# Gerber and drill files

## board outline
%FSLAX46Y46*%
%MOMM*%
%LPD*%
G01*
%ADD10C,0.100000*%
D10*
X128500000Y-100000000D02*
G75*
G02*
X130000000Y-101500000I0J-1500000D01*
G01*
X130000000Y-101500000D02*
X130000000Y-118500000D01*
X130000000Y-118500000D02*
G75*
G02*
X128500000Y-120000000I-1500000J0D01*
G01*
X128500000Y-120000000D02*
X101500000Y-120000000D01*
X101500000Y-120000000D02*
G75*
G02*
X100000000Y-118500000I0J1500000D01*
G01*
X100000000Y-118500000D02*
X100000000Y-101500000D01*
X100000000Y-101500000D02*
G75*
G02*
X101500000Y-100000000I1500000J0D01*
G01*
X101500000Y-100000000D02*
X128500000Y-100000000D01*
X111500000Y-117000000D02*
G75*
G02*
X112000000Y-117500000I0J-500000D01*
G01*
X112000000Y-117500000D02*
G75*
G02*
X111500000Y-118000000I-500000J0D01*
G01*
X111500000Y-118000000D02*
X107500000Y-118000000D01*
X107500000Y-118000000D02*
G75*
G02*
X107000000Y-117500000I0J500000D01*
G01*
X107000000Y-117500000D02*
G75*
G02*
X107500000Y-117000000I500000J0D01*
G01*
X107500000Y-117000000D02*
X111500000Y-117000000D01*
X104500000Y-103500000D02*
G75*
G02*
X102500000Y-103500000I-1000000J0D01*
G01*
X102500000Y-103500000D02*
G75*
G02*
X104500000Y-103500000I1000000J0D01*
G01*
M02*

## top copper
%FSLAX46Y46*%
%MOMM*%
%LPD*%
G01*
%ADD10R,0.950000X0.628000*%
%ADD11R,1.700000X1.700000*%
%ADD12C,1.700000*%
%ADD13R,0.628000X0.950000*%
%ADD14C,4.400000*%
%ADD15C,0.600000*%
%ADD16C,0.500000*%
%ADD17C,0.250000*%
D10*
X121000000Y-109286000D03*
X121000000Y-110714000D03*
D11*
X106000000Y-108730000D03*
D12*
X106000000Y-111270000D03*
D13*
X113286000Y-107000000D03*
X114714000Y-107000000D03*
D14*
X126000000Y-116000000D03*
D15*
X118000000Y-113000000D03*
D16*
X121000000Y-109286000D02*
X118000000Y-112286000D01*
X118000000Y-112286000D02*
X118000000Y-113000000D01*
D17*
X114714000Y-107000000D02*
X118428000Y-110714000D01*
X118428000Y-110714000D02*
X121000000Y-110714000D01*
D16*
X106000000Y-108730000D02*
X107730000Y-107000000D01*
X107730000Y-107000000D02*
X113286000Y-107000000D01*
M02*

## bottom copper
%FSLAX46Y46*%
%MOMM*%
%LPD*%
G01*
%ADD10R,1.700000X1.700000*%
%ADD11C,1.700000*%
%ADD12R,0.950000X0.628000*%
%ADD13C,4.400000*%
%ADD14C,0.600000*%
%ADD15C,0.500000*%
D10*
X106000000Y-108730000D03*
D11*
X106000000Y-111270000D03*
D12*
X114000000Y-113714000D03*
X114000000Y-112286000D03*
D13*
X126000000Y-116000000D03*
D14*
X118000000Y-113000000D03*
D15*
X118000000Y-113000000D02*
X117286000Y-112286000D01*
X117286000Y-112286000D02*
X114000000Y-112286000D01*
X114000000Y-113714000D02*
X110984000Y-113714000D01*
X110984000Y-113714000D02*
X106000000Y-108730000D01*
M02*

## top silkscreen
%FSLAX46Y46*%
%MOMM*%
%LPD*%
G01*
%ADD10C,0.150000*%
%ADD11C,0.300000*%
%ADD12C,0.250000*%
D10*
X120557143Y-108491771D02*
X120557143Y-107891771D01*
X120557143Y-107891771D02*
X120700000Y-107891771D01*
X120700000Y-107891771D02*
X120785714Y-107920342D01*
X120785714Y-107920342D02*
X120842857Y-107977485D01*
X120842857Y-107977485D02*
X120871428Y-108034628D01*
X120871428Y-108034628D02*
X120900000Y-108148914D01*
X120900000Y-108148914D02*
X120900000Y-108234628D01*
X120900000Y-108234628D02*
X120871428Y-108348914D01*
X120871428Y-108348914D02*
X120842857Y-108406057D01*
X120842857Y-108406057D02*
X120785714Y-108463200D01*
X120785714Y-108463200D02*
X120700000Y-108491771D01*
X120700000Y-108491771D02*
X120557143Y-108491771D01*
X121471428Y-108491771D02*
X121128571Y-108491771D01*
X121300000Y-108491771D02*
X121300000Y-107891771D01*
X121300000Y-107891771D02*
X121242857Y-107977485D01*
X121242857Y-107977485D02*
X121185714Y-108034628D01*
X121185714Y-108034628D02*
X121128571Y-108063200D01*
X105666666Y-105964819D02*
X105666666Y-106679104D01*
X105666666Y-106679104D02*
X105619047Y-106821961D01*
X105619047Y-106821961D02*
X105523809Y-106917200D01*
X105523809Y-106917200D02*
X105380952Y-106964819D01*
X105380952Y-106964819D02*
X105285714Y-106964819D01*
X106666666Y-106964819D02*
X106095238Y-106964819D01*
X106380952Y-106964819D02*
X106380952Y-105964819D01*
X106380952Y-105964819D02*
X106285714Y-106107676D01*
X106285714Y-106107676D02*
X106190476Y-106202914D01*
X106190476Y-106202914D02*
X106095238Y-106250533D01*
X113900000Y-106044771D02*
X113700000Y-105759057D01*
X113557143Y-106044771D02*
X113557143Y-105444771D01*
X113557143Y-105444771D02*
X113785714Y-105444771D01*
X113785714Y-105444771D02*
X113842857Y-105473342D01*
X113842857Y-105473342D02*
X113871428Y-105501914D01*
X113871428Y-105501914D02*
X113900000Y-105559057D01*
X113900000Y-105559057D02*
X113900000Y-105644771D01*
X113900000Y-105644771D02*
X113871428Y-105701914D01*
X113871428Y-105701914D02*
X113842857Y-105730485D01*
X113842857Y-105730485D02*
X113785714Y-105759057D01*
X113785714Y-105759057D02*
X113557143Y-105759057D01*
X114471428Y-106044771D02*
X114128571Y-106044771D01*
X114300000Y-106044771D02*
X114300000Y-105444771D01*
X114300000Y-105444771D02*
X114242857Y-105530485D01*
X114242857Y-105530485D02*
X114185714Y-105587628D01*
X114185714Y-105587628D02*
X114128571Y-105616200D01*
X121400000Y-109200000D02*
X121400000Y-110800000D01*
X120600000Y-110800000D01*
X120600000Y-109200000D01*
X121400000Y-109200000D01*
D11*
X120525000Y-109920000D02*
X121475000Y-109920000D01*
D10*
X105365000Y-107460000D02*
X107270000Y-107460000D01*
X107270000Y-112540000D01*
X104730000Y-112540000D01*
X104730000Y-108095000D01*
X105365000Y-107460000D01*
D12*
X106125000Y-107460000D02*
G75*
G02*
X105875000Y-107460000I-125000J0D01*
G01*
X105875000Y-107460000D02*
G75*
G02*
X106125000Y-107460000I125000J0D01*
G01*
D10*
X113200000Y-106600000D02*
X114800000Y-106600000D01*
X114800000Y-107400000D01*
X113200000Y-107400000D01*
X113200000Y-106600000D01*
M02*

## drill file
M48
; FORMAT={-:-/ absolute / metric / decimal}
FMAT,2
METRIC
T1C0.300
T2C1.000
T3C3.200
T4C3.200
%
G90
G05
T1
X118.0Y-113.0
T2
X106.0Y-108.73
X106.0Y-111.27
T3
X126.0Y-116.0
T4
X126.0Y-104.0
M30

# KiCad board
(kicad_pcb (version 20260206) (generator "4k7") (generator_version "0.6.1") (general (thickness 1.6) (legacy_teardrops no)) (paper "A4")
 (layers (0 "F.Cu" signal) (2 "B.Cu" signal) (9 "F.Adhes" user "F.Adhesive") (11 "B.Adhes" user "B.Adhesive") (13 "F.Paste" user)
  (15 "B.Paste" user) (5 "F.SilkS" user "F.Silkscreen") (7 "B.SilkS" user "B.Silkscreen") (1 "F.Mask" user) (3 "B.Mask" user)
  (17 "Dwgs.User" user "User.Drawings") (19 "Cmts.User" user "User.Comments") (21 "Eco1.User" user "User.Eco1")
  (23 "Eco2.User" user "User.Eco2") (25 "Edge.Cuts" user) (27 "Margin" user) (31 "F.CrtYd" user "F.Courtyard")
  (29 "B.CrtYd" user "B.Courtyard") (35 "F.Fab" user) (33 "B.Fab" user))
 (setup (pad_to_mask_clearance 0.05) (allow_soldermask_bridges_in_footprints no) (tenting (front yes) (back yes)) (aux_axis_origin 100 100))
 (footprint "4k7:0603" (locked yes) (layer "F.Cu") (at 121 110 -90)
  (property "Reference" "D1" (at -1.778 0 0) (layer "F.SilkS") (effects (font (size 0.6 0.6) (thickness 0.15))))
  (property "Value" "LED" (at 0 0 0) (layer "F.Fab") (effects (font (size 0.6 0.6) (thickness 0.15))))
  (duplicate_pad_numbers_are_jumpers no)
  (fp_poly (pts (xy -0.8 -0.4) (xy 0.8 -0.4) (xy 0.8 0.4) (xy -0.8 0.4)) (stroke (width 0.15) (type solid)) (fill no) (layer "F.SilkS"))
  (fp_line (start -0.08 0.475) (end -0.08 -0.475) (stroke (width 0.3) (type solid)) (layer "F.SilkS"))
  (pad "1" smd rect (at -0.714 0 -90) (size 0.628 0.95) (layers "F.Cu" "F.Mask" "F.Paste") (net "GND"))
  (pad "2" smd rect (at 0.714 0 -90) (size 0.628 0.95) (layers "F.Cu" "F.Mask" "F.Paste") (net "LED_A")))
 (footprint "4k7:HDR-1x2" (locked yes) (layer "F.Cu") (at 106 110)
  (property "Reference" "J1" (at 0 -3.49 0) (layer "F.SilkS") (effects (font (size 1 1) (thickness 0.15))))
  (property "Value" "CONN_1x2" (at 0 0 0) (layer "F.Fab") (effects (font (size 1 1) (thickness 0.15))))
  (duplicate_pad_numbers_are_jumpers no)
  (fp_poly
   (pts (xy -0.635 -2.54) (xy 1.27 -2.54) (xy 1.27 2.54) (xy -1.27 2.54) (xy -1.27 -1.905)) (stroke (width 0.15) (type solid)) (fill no)
   (layer "F.SilkS"))
  (fp_circle (center 0 -2.54) (end 0.25 -2.54) (stroke (width 0) (type solid)) (fill yes) (layer "F.SilkS"))
  (pad "1" thru_hole rect (at 0 -1.27) (size 1.7 1.7) (drill 1) (layers "*.Cu" "*.Mask") (remove_unused_layers no) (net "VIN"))
  (pad "2" thru_hole circle (at 0 1.27) (size 1.7 1.7) (drill 1) (layers "*.Cu" "*.Mask") (remove_unused_layers no) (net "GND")))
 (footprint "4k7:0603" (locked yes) (layer "F.Cu") (at 114 107)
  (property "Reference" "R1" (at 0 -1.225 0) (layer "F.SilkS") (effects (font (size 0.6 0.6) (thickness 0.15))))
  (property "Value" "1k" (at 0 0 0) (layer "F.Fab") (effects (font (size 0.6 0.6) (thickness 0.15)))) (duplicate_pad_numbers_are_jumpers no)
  (fp_poly (pts (xy -0.8 -0.4) (xy 0.8 -0.4) (xy 0.8 0.4) (xy -0.8 0.4)) (stroke (width 0.15) (type solid)) (fill no) (layer "F.SilkS"))
  (pad "1" smd rect (at -0.714 0) (size 0.628 0.95) (layers "F.Cu" "F.Mask" "F.Paste") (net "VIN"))
  (pad "2" smd rect (at 0.714 0) (size 0.628 0.95) (layers "F.Cu" "F.Mask" "F.Paste") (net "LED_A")))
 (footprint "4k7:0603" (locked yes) (layer "B.Cu") (at 114 113 90)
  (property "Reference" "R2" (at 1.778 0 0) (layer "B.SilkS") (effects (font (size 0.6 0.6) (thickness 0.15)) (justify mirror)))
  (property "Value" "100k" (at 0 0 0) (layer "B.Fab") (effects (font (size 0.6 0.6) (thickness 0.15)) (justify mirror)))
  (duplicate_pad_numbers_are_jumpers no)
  (pad "1" smd rect (at -0.714 0 90) (size 0.628 0.95) (layers "B.Cu" "B.Mask" "B.Paste") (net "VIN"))
  (pad "2" smd rect (at 0.714 0 90) (size 0.628 0.95) (layers "B.Cu" "B.Mask" "B.Paste") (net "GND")))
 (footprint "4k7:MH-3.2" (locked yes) (layer "F.Cu") (at 126 104)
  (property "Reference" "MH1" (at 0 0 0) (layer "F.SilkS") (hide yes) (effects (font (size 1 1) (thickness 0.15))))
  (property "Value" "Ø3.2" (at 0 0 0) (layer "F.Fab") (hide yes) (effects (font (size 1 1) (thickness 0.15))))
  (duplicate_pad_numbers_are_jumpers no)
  (pad "1" np_thru_hole circle (at 0 0) (size 3.2 3.2) (drill 3.2) (layers "*.Cu" "*.Mask")))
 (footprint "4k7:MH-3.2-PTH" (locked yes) (layer "F.Cu") (at 126 116)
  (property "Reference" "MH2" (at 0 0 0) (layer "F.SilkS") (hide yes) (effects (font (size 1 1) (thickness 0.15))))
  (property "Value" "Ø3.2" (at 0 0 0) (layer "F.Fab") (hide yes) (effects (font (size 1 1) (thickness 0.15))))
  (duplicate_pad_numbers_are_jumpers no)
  (pad "1" thru_hole circle (at 0 0) (size 4.4 4.4) (drill 3.2) (layers "*.Cu" "*.Mask") (remove_unused_layers no) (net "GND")))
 (gr_arc (start 128.5 100) (mid 129.56066 100.43934) (end 130 101.5) (stroke (width 0.1) (type solid)) (layer "Edge.Cuts"))
 (gr_line (start 130 101.5) (end 130 118.5) (stroke (width 0.1) (type solid)) (layer "Edge.Cuts"))
 (gr_arc (start 130 118.5) (mid 129.56066 119.56066) (end 128.5 120) (stroke (width 0.1) (type solid)) (layer "Edge.Cuts"))
 (gr_line (start 128.5 120) (end 101.5 120) (stroke (width 0.1) (type solid)) (layer "Edge.Cuts"))
 (gr_arc (start 101.5 120) (mid 100.43934 119.56066) (end 100 118.5) (stroke (width 0.1) (type solid)) (layer "Edge.Cuts"))
 (gr_line (start 100 118.5) (end 100 101.5) (stroke (width 0.1) (type solid)) (layer "Edge.Cuts"))
 (gr_arc (start 100 101.5) (mid 100.43934 100.43934) (end 101.5 100) (stroke (width 0.1) (type solid)) (layer "Edge.Cuts"))
 (gr_line (start 101.5 100) (end 128.5 100) (stroke (width 0.1) (type solid)) (layer "Edge.Cuts"))
 (gr_arc (start 111.5 117) (mid 111.853553 117.146447) (end 112 117.5) (stroke (width 0.1) (type solid)) (layer "Edge.Cuts"))
 (gr_arc (start 112 117.5) (mid 111.853553 117.853553) (end 111.5 118) (stroke (width 0.1) (type solid)) (layer "Edge.Cuts"))
 (gr_line (start 111.5 118) (end 107.5 118) (stroke (width 0.1) (type solid)) (layer "Edge.Cuts"))
 (gr_arc (start 107.5 118) (mid 107.146447 117.853553) (end 107 117.5) (stroke (width 0.1) (type solid)) (layer "Edge.Cuts"))
 (gr_arc (start 107 117.5) (mid 107.146447 117.146447) (end 107.5 117) (stroke (width 0.1) (type solid)) (layer "Edge.Cuts"))
 (gr_line (start 107.5 117) (end 111.5 117) (stroke (width 0.1) (type solid)) (layer "Edge.Cuts"))
 (gr_circle (center 103.5 103.5) (end 104.5 103.5) (stroke (width 0.1) (type solid)) (fill no) (layer "Edge.Cuts"))
 (segment (start 121 109.286) (end 118 112.286) (width 0.5) (layer "F.Cu") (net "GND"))
 (segment (start 118 112.286) (end 118 113) (width 0.5) (layer "F.Cu") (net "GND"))
 (segment (start 118 113) (end 117.286 112.286) (width 0.5) (layer "B.Cu") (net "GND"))
 (segment (start 117.286 112.286) (end 114 112.286) (width 0.5) (layer "B.Cu") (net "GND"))
 (segment (start 114.714 107) (end 118.428 110.714) (width 0.25) (layer "F.Cu") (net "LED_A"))
 (segment (start 118.428 110.714) (end 121 110.714) (width 0.25) (layer "F.Cu") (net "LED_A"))
 (segment (start 106 108.73) (end 107.73 107) (width 0.5) (layer "F.Cu") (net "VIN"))
 (segment (start 107.73 107) (end 113.286 107) (width 0.5) (layer "F.Cu") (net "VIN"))
 (segment (start 114 113.714) (end 110.984 113.714) (width 0.5) (layer "B.Cu") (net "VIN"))
 (segment (start 110.984 113.714) (end 106 108.73) (width 0.5) (layer "B.Cu") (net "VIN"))
 (via (at 118 113) (size 0.6) (drill 0.3) (layers "F.Cu" "B.Cu") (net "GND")))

